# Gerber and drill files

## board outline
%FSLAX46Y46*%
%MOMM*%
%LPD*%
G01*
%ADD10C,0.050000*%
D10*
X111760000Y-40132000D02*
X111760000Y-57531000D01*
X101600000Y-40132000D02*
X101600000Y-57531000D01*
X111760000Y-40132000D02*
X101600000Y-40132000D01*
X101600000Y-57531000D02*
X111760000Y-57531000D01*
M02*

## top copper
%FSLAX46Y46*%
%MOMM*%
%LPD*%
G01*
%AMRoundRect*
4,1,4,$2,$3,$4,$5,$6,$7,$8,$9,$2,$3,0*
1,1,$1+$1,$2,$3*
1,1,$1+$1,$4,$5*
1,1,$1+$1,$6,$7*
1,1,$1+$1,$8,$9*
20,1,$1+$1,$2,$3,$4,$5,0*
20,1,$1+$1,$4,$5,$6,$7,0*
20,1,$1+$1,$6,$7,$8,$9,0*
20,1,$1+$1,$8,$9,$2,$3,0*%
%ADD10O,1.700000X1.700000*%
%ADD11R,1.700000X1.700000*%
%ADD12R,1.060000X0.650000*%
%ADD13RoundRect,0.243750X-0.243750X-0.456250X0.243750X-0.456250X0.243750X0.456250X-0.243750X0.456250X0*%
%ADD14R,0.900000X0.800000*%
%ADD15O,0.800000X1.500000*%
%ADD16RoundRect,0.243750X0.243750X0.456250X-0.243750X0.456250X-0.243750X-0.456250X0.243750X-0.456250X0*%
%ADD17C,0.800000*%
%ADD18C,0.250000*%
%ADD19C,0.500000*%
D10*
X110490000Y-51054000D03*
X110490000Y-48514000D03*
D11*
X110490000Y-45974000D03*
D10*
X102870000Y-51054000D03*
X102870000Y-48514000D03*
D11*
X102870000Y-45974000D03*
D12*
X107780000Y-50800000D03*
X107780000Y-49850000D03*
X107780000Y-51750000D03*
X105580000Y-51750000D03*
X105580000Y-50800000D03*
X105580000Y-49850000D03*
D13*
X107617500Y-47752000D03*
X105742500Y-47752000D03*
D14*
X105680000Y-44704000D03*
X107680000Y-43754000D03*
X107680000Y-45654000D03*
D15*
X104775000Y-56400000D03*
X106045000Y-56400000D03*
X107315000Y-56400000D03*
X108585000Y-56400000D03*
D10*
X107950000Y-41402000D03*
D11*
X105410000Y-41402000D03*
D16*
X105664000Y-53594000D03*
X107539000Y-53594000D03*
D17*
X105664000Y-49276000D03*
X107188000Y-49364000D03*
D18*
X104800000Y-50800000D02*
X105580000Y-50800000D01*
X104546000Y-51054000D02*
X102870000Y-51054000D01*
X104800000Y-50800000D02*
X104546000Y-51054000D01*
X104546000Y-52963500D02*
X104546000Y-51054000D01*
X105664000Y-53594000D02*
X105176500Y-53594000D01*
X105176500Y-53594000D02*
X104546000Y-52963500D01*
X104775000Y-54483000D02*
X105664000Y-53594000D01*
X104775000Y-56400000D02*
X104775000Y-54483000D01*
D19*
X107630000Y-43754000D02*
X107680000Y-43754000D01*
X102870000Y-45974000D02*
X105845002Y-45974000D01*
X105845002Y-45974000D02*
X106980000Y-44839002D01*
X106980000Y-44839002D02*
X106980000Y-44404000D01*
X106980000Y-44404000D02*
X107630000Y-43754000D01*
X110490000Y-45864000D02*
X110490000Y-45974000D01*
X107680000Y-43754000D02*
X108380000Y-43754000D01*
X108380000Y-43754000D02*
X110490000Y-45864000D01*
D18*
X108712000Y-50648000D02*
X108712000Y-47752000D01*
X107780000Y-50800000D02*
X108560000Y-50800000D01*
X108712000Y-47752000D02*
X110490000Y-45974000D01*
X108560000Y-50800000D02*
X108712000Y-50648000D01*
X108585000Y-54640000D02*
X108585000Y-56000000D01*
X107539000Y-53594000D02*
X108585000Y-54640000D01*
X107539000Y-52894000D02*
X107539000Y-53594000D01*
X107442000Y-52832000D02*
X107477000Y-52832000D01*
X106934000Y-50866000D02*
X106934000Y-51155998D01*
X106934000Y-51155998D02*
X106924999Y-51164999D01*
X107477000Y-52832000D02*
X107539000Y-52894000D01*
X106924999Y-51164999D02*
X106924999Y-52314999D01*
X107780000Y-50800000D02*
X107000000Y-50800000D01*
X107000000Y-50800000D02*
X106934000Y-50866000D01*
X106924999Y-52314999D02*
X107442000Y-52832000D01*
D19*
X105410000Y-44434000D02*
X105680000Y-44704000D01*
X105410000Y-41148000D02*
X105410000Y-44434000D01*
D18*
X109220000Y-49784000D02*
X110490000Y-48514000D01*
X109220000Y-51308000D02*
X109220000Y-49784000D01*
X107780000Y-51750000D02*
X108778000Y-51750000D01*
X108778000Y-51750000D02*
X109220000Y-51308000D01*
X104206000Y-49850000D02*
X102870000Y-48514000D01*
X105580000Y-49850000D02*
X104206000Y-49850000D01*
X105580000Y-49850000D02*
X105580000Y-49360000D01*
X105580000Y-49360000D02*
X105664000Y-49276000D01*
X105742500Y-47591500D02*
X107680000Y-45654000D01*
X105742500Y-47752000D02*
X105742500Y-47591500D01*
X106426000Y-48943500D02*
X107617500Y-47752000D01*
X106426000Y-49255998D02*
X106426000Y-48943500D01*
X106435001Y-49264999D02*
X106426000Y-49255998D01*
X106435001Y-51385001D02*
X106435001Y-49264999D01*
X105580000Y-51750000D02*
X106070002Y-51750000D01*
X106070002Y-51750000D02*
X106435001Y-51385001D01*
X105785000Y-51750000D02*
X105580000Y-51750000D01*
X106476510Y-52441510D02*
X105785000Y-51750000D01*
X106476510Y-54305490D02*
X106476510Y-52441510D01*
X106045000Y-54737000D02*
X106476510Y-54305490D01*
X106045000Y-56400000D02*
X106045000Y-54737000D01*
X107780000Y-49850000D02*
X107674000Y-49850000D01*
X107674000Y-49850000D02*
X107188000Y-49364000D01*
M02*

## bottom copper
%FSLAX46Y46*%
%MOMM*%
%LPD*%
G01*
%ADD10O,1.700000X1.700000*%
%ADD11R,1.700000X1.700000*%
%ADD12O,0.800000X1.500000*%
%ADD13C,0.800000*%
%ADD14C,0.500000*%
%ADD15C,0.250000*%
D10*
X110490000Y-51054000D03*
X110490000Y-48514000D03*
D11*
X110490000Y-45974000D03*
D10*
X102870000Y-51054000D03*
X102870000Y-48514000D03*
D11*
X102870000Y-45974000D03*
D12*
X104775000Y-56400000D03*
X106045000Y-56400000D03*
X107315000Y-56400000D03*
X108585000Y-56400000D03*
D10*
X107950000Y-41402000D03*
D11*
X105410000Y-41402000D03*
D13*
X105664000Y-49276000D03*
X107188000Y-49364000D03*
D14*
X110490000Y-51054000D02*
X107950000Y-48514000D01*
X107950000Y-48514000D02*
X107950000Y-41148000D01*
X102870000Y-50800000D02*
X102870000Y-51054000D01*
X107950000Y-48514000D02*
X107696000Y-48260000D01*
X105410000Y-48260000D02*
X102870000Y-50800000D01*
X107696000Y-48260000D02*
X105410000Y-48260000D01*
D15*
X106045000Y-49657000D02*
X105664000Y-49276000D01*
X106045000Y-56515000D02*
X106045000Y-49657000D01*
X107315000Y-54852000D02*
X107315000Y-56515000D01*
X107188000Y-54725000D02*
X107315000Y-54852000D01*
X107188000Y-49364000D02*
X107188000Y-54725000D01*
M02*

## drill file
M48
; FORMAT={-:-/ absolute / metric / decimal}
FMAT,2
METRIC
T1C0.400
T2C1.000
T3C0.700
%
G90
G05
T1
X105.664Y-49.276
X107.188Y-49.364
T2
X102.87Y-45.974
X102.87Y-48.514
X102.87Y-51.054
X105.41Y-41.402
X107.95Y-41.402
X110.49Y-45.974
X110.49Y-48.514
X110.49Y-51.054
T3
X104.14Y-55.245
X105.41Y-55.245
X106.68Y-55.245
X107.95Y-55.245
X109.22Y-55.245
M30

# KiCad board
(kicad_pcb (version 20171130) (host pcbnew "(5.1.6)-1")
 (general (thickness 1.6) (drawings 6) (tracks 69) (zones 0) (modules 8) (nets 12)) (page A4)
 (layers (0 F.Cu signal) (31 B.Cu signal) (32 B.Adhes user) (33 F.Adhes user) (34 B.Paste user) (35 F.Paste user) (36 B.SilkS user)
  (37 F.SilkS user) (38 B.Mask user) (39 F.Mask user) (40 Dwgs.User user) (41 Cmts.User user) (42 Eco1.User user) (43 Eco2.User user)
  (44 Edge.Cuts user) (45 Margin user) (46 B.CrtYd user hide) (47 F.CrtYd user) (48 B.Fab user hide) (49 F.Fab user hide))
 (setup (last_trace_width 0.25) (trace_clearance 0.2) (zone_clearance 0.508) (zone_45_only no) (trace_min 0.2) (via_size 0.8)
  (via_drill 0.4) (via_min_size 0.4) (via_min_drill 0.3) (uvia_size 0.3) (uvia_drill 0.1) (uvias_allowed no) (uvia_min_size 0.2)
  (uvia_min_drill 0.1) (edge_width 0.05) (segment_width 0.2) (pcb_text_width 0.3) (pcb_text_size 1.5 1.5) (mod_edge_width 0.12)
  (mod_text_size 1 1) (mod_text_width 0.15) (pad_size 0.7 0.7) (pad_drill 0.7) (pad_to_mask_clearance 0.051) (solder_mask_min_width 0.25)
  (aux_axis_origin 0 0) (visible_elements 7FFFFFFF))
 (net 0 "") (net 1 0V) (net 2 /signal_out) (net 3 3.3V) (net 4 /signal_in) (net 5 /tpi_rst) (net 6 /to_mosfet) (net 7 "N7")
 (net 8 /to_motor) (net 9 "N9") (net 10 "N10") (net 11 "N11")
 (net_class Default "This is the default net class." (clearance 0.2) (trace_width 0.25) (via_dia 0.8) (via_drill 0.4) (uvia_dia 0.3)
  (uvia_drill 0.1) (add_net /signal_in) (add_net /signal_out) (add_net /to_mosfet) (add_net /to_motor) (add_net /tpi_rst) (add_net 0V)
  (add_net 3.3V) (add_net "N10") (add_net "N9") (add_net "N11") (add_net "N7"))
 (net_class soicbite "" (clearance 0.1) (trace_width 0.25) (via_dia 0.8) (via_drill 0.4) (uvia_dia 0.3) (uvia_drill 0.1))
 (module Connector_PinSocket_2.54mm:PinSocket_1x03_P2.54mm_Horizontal (layer B.Cu) (at 110.49 45.974 180)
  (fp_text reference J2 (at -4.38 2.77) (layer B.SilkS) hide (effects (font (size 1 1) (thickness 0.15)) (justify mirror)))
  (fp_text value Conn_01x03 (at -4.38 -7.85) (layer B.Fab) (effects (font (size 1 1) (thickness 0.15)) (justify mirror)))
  (pad 3 thru_hole oval (at 0 -5.08 180) (size 1.7 1.7) (drill 1) (layers *.Cu *.Mask) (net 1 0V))
  (pad 2 thru_hole oval (at 0 -2.54 180) (size 1.7 1.7) (drill 1) (layers *.Cu *.Mask) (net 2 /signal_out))
  (pad 1 thru_hole rect (at 0 0 180) (size 1.7 1.7) (drill 1) (layers *.Cu *.Mask) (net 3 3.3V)))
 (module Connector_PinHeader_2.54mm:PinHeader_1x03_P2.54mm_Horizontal (layer B.Cu) (at 102.87 45.974 180)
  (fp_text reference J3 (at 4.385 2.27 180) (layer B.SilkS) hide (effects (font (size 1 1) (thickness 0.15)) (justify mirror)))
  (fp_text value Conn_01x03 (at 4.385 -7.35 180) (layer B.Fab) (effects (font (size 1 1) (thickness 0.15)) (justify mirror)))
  (pad 3 thru_hole oval (at 0 -5.08 180) (size 1.7 1.7) (drill 1) (layers *.Cu *.Mask) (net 1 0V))
  (pad 2 thru_hole oval (at 0 -2.54 180) (size 1.7 1.7) (drill 1) (layers *.Cu *.Mask) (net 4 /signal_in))
  (pad 1 thru_hole rect (at 0 0 180) (size 1.7 1.7) (drill 1) (layers *.Cu *.Mask) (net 3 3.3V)))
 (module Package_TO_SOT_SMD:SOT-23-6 (layer F.Cu) (at 106.68 50.8)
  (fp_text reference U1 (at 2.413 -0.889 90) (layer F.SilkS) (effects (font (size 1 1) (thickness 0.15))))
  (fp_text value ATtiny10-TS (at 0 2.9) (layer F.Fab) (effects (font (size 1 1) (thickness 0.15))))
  (pad 5 smd rect (at 1.1 0) (size 1.06 0.65) (layers F.Cu F.Paste F.Mask) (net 3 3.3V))
  (pad 6 smd rect (at 1.1 -0.95) (size 1.06 0.65) (layers F.Cu F.Paste F.Mask) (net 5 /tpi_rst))
  (pad 4 smd rect (at 1.1 0.95) (size 1.06 0.65) (layers F.Cu F.Paste F.Mask) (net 2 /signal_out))
  (pad 3 smd rect (at -1.1 0.95) (size 1.06 0.65) (layers F.Cu F.Paste F.Mask) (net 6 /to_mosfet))
  (pad 2 smd rect (at -1.1 0) (size 1.06 0.65) (layers F.Cu F.Paste F.Mask) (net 1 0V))
  (pad 1 smd rect (at -1.1 -0.95) (size 1.06 0.65) (layers F.Cu F.Paste F.Mask) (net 4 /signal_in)))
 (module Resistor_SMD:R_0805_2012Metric (layer F.Cu) (at 106.68 47.752)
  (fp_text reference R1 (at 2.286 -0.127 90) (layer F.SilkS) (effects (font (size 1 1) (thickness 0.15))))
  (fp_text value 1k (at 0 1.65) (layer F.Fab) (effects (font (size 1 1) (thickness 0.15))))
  (pad 2 smd roundrect (at 0.9375 0) (size 0.975 1.4) (layers F.Cu F.Paste F.Mask) (roundrect_rratio 0.25) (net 6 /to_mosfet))
  (pad 1 smd roundrect (at -0.9375 0) (size 0.975 1.4) (layers F.Cu F.Paste F.Mask) (roundrect_rratio 0.25) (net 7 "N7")))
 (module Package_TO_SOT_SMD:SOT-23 (layer F.Cu) (at 106.68 44.704 180)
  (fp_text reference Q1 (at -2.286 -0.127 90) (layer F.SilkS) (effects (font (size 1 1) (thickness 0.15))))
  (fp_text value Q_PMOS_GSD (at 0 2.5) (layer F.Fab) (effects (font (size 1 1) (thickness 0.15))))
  (pad 3 smd rect (at 1 0 180) (size 0.9 0.8) (layers F.Cu F.Paste F.Mask) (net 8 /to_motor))
  (pad 2 smd rect (at -1 0.95 180) (size 0.9 0.8) (layers F.Cu F.Paste F.Mask) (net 3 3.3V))
  (pad 1 smd rect (at -1 -0.95 180) (size 0.9 0.8) (layers F.Cu F.Paste F.Mask) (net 7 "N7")))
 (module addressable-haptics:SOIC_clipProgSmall (layer F.Cu) (at 106.68 57.15)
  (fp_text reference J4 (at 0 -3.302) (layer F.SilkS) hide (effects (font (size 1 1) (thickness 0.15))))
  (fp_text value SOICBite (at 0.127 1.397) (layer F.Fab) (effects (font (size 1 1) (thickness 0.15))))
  (pad 5 smd oval (at -1.905 -0.75) (size 0.8 1.5) (layers B.Cu B.Mask) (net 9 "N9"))
  (pad 4 smd oval (at -1.905 -0.75) (size 0.8 1.5) (layers F.Cu F.Mask) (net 1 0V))
  (pad 3 smd oval (at -0.635 -0.75) (size 0.8 1.5) (layers F.Cu F.Mask) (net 6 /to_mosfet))
  (pad 2 smd oval (at 0.635 -0.75) (size 0.8 1.5) (layers F.Cu F.Mask) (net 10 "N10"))
  (pad 1 smd oval (at 1.905 -0.75) (size 0.8 1.5) (layers F.Cu F.Mask) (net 3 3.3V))
  (pad 6 smd oval (at -0.635 -0.75) (size 0.8 1.5) (layers B.Cu B.Mask) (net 4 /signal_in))
  (pad 7 smd oval (at 0.635 -0.75) (size 0.8 1.5) (layers B.Cu B.Mask) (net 5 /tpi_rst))
  (pad 8 smd oval (at 1.905 -0.75) (size 0.8 1.5) (layers B.Cu B.Mask) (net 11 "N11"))
  (pad "" np_thru_hole circle (at -2.54 -1.905) (size 0.7 0.7) (drill 0.7) (layers *.Cu *.Mask) (clearance 0.1))
  (pad "" np_thru_hole circle (at -1.27 -1.905) (size 0.7 0.7) (drill 0.7) (layers *.Cu *.Mask) (clearance 0.1))
  (pad "" np_thru_hole circle (at 0 -1.905) (size 0.7 0.7) (drill 0.7) (layers *.Cu *.Mask) (clearance 0.1))
  (pad "" np_thru_hole circle (at 1.27 -1.905) (size 0.7 0.7) (drill 0.7) (layers *.Cu *.Mask) (clearance 0.1))
  (pad "" np_thru_hole circle (at 2.54 -1.905) (size 0.7 0.7) (drill 0.7) (layers *.Cu *.Mask) (clearance 0.1)))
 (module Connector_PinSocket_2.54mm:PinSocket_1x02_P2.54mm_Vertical (layer F.Cu) (at 105.41 41.402 90)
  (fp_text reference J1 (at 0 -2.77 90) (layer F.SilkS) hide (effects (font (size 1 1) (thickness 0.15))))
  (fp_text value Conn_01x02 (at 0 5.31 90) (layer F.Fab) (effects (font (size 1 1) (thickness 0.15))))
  (pad 2 thru_hole oval (at 0 2.54 90) (size 1.7 1.7) (drill 1) (layers *.Cu *.Mask) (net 1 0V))
  (pad 1 thru_hole rect (at 0 0 90) (size 1.7 1.7) (drill 1) (layers *.Cu *.Mask) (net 8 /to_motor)))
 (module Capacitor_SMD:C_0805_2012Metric (layer F.Cu) (at 106.6015 53.594 180)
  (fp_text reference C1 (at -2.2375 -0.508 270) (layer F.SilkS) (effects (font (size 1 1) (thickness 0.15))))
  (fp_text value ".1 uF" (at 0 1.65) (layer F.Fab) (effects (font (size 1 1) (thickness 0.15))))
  (pad 2 smd roundrect (at 0.9375 0 180) (size 0.975 1.4) (layers F.Cu F.Paste F.Mask) (roundrect_rratio 0.25) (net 1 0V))
  (pad 1 smd roundrect (at -0.9375 0 180) (size 0.975 1.4) (layers F.Cu F.Paste F.Mask) (roundrect_rratio 0.25) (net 3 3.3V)))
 (gr_line (start 111.76 40.132) (end 111.76 57.531) (layer Edge.Cuts) (width 0.05))
 (gr_line (start 101.6 40.132) (end 101.6 57.531) (layer Edge.Cuts) (width 0.05))
 (gr_line (start 111.76 40.132) (end 101.6 40.132) (layer Edge.Cuts) (width 0.05))
 (gr_line (start 101.6 57.531) (end 111.76 57.531) (layer Edge.Cuts) (width 0.05))
 (segment (start 104.8 50.8) (end 105.58 50.8) (width 0.25) (layer F.Cu) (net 1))
 (segment (start 104.546 51.054) (end 102.87 51.054) (width 0.25) (layer F.Cu) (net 1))
 (segment (start 104.8 50.8) (end 104.546 51.054) (width 0.25) (layer F.Cu) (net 1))
 (segment (start 104.546 52.9635) (end 104.546 51.054) (width 0.25) (layer F.Cu) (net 1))
 (segment (start 105.664 53.594) (end 105.1765 53.594) (width 0.25) (layer F.Cu) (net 1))
 (segment (start 105.1765 53.594) (end 104.546 52.9635) (width 0.25) (layer F.Cu) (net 1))
 (segment (start 110.49 51.054) (end 107.95 48.514) (width 0.5) (layer B.Cu) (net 1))
 (segment (start 107.95 48.514) (end 107.95 41.148) (width 0.5) (layer B.Cu) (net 1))
 (segment (start 104.775 54.483) (end 105.664 53.594) (width 0.25) (layer F.Cu) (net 1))
 (segment (start 104.775 56.4) (end 104.775 54.483) (width 0.25) (layer F.Cu) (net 1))
 (segment (start 102.87 50.8) (end 102.87 51.054) (width 0.5) (layer B.Cu) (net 1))
 (segment (start 107.95 48.514) (end 107.696 48.26) (width 0.5) (layer B.Cu) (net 1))
 (segment (start 105.41 48.26) (end 102.87 50.8) (width 0.5) (layer B.Cu) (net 1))
 (segment (start 107.696 48.26) (end 105.41 48.26) (width 0.5) (layer B.Cu) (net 1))
 (segment (start 107.63 43.754) (end 107.68 43.754) (width 0.5) (layer F.Cu) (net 3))
 (segment (start 102.87 45.974) (end 105.845002 45.974) (width 0.5) (layer F.Cu) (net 3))
 (segment (start 105.845002 45.974) (end 106.98 44.839002) (width 0.5) (layer F.Cu) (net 3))
 (segment (start 106.98 44.839002) (end 106.98 44.404) (width 0.5) (layer F.Cu) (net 3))
 (segment (start 106.98 44.404) (end 107.63 43.754) (width 0.5) (layer F.Cu) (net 3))
 (segment (start 110.49 45.864) (end 110.49 45.974) (width 0.5) (layer F.Cu) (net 3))
 (segment (start 107.68 43.754) (end 108.38 43.754) (width 0.5) (layer F.Cu) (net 3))
 (segment (start 108.38 43.754) (end 110.49 45.864) (width 0.5) (layer F.Cu) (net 3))
 (segment (start 108.712 50.648) (end 108.712 47.752) (width 0.25) (layer F.Cu) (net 3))
 (segment (start 107.78 50.8) (end 108.56 50.8) (width 0.25) (layer F.Cu) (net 3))
 (segment (start 108.712 47.752) (end 110.49 45.974) (width 0.25) (layer F.Cu) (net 3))
 (segment (start 108.56 50.8) (end 108.712 50.648) (width 0.25) (layer F.Cu) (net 3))
 (segment (start 108.585 54.64) (end 108.585 56) (width 0.25) (layer F.Cu) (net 3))
 (segment (start 107.539 53.594) (end 108.585 54.64) (width 0.25) (layer F.Cu) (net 3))
 (segment (start 107.539 52.894) (end 107.539 53.594) (width 0.25) (layer F.Cu) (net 3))
 (segment (start 107.442 52.832) (end 107.477 52.832) (width 0.25) (layer F.Cu) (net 3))
 (segment (start 106.934 50.866) (end 106.934 51.155998) (width 0.25) (layer F.Cu) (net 3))
 (segment (start 106.934 51.155998) (end 106.924999 51.164999) (width 0.25) (layer F.Cu) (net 3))
 (segment (start 107.477 52.832) (end 107.539 52.894) (width 0.25) (layer F.Cu) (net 3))
 (segment (start 106.924999 51.164999) (end 106.924999 52.314999) (width 0.25) (layer F.Cu) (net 3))
 (segment (start 107.78 50.8) (end 107 50.8) (width 0.25) (layer F.Cu) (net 3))
 (segment (start 107 50.8) (end 106.934 50.866) (width 0.25) (layer F.Cu) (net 3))
 (segment (start 106.924999 52.314999) (end 107.442 52.832) (width 0.25) (layer F.Cu) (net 3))
 (segment (start 105.41 44.434) (end 105.68 44.704) (width 0.5) (layer F.Cu) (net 8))
 (segment (start 105.41 41.148) (end 105.41 44.434) (width 0.5) (layer F.Cu) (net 8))
 (segment (start 109.22 49.784) (end 110.49 48.514) (width 0.25) (layer F.Cu) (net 2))
 (segment (start 109.22 51.308) (end 109.22 49.784) (width 0.25) (layer F.Cu) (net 2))
 (segment (start 107.78 51.75) (end 108.778 51.75) (width 0.25) (layer F.Cu) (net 2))
 (segment (start 108.778 51.75) (end 109.22 51.308) (width 0.25) (layer F.Cu) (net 2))
 (segment (start 104.206 49.85) (end 102.87 48.514) (width 0.25) (layer F.Cu) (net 4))
 (segment (start 105.58 49.85) (end 104.206 49.85) (width 0.25) (layer F.Cu) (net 4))
 (via (at 105.664 49.276) (size 0.8) (drill 0.4) (layers F.Cu B.Cu) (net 4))
 (segment (start 105.58 49.85) (end 105.58 49.36) (width 0.25) (layer F.Cu) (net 4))
 (segment (start 105.58 49.36) (end 105.664 49.276) (width 0.25) (layer F.Cu) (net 4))
 (segment (start 106.045 49.657) (end 105.664 49.276) (width 0.25) (layer B.Cu) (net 4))
 (segment (start 106.045 56.515) (end 106.045 49.657) (width 0.25) (layer B.Cu) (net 4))
 (segment (start 105.7425 47.5915) (end 107.68 45.654) (width 0.25) (layer F.Cu) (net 7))
 (segment (start 105.7425 47.752) (end 105.7425 47.5915) (width 0.25) (layer F.Cu) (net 7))
 (segment (start 106.426 48.9435) (end 107.6175 47.752) (width 0.25) (layer F.Cu) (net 6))
 (segment (start 106.426 49.255998) (end 106.426 48.9435) (width 0.25) (layer F.Cu) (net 6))
 (segment (start 106.435001 49.264999) (end 106.426 49.255998) (width 0.25) (layer F.Cu) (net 6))
 (segment (start 106.435001 51.385001) (end 106.435001 49.264999) (width 0.25) (layer F.Cu) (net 6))
 (segment (start 105.58 51.75) (end 106.070002 51.75) (width 0.25) (layer F.Cu) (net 6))
 (segment (start 106.070002 51.75) (end 106.435001 51.385001) (width 0.25) (layer F.Cu) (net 6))
 (segment (start 105.785 51.75) (end 105.58 51.75) (width 0.25) (layer F.Cu) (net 6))
 (segment (start 106.47651 52.44151) (end 105.785 51.75) (width 0.25) (layer F.Cu) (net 6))
 (segment (start 106.47651 54.30549) (end 106.47651 52.44151) (width 0.25) (layer F.Cu) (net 6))
 (segment (start 106.045 54.737) (end 106.47651 54.30549) (width 0.25) (layer F.Cu) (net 6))
 (segment (start 106.045 56.4) (end 106.045 54.737) (width 0.25) (layer F.Cu) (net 6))
 (segment (start 107.315 54.852) (end 107.315 56.515) (width 0.25) (layer B.Cu) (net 5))
 (via (at 107.188 49.364) (size 0.8) (drill 0.4) (layers F.Cu B.Cu) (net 5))
 (segment (start 107.78 49.85) (end 107.674 49.85) (width 0.25) (layer F.Cu) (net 5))
 (segment (start 107.674 49.85) (end 107.188 49.364) (width 0.25) (layer F.Cu) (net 5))
 (segment (start 107.188 54.725) (end 107.315 54.852) (width 0.25) (layer B.Cu) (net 5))
 (segment (start 107.188 49.364) (end 107.188 54.725) (width 0.25) (layer B.Cu) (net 5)))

